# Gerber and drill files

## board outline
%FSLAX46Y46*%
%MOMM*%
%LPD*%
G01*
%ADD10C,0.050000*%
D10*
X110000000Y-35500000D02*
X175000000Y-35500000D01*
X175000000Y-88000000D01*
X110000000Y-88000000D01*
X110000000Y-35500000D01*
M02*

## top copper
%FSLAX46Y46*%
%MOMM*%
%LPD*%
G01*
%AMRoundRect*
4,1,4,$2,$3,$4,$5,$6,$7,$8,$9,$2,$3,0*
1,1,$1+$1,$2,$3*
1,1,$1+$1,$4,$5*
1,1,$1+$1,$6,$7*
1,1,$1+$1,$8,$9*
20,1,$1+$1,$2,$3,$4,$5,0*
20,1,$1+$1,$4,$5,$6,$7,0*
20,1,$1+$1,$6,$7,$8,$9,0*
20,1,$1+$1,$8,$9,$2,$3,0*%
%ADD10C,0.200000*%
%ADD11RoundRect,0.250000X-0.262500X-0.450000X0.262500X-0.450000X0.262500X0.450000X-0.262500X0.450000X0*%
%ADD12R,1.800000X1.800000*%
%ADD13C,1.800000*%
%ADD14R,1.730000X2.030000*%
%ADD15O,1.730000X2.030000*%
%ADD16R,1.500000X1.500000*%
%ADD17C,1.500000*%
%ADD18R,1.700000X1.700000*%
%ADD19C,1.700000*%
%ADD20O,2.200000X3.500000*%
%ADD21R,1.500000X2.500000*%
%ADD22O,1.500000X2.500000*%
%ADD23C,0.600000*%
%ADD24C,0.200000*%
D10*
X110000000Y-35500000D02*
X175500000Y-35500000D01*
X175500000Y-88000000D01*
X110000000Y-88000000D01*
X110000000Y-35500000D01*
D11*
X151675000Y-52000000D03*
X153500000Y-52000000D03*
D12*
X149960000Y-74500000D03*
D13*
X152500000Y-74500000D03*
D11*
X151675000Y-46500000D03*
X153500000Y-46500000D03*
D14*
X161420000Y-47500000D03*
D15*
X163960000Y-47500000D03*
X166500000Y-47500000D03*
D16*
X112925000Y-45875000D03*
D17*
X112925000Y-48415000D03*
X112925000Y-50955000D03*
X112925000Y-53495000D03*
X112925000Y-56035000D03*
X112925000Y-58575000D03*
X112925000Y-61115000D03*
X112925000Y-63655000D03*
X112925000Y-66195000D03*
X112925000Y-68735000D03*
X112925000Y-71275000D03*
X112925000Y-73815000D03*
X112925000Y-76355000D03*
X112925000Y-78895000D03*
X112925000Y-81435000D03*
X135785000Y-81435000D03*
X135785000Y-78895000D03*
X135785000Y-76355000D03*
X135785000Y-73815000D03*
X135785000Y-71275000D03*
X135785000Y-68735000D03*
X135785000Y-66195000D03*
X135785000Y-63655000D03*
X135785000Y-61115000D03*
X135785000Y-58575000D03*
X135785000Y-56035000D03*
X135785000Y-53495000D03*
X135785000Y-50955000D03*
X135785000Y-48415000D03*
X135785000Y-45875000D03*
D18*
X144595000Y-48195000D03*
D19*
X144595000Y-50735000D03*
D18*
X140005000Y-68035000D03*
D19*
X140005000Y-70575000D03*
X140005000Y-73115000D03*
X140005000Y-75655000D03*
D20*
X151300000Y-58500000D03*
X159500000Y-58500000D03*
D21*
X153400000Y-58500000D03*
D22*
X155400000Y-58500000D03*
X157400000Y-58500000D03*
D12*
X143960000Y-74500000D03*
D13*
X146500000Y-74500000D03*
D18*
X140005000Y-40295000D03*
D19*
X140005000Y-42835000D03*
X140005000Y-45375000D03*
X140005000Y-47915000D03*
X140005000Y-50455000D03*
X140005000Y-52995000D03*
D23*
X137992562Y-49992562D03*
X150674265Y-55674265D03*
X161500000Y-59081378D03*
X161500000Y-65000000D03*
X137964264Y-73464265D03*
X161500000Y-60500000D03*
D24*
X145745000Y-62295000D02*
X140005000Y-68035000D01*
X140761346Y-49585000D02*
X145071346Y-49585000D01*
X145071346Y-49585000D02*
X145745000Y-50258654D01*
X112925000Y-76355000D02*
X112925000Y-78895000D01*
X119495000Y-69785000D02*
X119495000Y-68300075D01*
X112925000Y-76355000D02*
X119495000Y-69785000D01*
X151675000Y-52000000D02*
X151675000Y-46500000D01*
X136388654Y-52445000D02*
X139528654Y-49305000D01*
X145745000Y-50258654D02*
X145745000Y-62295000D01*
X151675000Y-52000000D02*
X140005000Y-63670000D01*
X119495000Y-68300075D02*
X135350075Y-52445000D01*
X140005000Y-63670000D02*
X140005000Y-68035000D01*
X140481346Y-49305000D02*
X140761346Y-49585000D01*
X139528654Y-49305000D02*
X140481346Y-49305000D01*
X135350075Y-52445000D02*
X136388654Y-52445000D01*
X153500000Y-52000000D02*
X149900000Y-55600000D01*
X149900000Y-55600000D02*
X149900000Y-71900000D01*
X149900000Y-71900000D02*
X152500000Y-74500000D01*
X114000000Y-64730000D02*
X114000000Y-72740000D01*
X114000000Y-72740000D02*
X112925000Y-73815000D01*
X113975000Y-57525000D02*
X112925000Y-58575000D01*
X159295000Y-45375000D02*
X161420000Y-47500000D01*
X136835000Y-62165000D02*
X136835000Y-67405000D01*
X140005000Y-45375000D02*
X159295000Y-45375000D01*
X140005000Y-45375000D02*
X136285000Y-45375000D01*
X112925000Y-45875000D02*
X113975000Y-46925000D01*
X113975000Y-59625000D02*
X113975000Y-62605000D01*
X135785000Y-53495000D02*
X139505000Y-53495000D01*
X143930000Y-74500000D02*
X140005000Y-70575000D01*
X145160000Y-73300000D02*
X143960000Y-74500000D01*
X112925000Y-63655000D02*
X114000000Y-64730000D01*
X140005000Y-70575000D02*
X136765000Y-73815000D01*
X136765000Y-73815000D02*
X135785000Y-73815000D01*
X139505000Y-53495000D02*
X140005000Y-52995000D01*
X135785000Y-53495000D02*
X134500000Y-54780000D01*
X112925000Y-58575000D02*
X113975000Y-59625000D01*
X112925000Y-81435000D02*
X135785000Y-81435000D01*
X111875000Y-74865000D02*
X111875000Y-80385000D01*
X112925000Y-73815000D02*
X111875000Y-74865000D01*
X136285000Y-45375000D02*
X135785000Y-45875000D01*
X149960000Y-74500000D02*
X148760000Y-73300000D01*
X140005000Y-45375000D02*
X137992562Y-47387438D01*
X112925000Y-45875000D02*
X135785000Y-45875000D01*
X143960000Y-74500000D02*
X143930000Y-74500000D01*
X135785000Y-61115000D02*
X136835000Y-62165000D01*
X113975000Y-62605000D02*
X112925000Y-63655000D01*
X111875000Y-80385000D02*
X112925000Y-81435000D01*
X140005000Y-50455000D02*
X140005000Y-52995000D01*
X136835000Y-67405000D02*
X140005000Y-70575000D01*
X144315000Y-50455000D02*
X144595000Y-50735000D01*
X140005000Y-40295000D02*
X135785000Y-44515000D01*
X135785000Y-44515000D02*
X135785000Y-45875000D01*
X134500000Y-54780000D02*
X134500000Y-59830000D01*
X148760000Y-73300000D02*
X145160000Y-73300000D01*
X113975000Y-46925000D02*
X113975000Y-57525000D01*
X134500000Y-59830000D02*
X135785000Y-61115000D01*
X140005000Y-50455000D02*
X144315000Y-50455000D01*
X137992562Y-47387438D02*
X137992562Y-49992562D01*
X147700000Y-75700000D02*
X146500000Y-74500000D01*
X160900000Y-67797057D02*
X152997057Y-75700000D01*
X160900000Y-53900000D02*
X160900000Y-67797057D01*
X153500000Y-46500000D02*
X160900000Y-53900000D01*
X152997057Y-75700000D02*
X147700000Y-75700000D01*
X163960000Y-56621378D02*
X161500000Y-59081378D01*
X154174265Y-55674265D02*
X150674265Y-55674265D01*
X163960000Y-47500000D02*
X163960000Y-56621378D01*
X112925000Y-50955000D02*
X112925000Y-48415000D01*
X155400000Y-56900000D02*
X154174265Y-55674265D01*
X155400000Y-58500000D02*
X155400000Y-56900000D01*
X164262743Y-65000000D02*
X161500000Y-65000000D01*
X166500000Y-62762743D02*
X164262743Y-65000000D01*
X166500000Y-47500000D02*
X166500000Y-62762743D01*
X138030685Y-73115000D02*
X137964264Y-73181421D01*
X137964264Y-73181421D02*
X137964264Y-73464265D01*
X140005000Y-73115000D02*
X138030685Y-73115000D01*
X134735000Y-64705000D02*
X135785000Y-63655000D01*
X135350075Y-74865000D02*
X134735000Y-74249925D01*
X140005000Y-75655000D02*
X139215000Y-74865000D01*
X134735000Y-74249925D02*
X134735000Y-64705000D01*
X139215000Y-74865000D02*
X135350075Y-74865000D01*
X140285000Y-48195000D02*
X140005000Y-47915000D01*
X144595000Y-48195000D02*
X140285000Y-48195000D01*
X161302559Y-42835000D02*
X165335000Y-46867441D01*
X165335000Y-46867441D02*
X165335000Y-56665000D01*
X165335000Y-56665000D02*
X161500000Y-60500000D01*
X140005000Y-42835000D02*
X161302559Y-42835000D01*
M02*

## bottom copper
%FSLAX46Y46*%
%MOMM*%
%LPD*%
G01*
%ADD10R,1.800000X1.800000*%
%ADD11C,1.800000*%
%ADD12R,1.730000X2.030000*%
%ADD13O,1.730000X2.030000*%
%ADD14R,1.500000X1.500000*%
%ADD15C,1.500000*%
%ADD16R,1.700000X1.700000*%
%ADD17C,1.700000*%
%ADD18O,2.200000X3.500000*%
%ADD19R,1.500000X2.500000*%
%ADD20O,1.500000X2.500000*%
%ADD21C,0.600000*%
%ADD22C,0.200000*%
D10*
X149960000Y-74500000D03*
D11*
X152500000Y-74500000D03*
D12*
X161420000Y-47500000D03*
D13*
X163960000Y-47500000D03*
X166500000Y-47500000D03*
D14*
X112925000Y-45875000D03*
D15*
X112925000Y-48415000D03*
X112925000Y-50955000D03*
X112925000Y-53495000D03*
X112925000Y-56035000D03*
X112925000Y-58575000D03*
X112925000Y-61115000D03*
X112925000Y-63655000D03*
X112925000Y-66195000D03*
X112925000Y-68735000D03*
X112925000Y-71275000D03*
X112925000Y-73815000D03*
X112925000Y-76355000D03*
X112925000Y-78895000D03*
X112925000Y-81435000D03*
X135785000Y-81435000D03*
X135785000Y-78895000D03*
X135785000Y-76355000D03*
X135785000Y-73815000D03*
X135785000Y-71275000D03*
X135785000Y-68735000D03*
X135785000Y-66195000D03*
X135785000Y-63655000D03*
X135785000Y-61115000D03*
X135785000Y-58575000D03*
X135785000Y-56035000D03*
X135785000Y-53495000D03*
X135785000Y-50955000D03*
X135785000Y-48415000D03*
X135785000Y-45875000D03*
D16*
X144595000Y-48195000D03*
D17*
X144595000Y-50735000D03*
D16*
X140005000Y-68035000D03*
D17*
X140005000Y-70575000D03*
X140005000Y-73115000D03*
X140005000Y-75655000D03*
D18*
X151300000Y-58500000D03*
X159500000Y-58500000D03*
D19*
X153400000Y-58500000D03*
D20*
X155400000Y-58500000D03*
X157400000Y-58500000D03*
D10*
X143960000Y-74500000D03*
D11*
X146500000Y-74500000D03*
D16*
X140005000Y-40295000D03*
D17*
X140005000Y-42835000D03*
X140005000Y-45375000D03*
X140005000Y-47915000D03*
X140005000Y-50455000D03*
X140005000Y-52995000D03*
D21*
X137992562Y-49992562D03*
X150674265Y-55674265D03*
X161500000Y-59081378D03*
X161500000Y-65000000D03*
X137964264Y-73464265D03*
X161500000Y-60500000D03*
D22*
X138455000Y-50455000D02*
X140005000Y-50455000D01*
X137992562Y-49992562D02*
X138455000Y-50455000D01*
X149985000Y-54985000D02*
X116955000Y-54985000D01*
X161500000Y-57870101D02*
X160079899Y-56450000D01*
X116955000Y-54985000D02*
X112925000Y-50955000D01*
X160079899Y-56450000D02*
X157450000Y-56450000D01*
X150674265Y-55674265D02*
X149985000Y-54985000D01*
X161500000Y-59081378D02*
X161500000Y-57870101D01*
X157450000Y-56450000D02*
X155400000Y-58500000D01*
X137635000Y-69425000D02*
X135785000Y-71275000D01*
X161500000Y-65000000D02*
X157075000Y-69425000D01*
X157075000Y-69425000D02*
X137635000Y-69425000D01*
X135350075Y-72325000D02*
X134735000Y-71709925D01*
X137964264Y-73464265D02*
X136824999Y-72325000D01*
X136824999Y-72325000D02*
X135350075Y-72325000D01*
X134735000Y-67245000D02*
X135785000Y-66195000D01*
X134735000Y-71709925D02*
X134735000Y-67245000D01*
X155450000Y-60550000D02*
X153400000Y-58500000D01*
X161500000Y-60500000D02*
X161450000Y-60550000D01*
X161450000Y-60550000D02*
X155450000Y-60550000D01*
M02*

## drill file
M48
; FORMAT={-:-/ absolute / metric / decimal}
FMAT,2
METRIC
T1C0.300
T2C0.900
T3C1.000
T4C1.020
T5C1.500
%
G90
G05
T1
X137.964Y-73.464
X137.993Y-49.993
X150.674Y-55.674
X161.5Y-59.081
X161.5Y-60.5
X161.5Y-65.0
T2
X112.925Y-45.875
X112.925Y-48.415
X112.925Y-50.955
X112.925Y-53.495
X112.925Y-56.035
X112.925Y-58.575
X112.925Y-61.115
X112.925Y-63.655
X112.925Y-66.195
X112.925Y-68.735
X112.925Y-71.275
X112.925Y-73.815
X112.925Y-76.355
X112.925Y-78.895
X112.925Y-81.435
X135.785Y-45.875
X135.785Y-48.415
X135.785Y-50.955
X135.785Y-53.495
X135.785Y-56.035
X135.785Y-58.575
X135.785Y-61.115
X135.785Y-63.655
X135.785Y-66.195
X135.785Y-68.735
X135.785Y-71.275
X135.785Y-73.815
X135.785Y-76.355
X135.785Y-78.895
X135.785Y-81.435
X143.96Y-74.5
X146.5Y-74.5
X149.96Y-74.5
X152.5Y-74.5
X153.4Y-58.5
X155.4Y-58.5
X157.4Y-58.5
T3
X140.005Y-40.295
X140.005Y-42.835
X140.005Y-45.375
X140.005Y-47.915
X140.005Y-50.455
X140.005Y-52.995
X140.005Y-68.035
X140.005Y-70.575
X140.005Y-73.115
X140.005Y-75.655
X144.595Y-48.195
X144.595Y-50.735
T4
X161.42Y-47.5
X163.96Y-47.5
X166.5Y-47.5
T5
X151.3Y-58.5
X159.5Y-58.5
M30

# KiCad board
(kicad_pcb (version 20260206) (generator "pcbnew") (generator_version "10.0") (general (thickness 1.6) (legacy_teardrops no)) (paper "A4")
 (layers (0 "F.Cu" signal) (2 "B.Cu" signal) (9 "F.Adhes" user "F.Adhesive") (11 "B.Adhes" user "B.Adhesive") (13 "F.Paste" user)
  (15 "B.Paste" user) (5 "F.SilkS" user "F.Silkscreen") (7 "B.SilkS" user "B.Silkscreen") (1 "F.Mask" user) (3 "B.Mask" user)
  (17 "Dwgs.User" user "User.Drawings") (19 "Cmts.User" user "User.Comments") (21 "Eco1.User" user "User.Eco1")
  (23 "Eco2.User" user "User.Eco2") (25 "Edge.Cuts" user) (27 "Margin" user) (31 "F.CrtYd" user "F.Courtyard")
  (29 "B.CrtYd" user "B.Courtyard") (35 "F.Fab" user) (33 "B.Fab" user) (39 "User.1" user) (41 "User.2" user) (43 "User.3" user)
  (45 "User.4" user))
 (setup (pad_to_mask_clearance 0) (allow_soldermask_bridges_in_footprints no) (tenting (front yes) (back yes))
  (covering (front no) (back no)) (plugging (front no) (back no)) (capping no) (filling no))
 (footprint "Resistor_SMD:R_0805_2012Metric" (layer "F.Cu") (at 152.5875 52)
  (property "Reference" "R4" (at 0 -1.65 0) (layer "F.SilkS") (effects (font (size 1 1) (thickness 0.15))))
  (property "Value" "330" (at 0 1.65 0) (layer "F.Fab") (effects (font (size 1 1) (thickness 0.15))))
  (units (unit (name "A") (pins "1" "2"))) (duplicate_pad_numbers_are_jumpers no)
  (pad "1" smd roundrect (at -0.9125 0) (size 1.025 1.4) (layers "F.Cu" "F.Mask" "F.Paste") (roundrect_rratio 0.243902) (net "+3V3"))
  (pad "2" smd roundrect (at 0.9125 0) (size 1.025 1.4) (layers "F.Cu" "F.Mask" "F.Paste") (roundrect_rratio 0.243902) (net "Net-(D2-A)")))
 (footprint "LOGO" (layer "F.Cu") (at 161.5 79)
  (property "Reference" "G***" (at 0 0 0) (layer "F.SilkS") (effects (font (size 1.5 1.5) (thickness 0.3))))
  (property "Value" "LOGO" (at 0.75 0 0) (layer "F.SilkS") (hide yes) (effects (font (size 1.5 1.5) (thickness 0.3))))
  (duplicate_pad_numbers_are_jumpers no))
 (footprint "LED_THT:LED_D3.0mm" (layer "F.Cu") (at 149.96 74.5)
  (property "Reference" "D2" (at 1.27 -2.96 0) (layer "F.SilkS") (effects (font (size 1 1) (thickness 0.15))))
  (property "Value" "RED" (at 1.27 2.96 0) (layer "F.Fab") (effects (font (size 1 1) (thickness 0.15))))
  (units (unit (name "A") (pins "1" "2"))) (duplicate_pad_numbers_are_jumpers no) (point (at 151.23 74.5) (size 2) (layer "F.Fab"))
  (pad "1" thru_hole rect (at 0 0) (size 1.8 1.8) (drill 0.9) (layers "*.Cu" "*.Mask") (remove_unused_layers no) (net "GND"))
  (pad "2" thru_hole circle (at 2.54 0) (size 1.8 1.8) (drill 0.9) (layers "*.Cu" "*.Mask") (remove_unused_layers no) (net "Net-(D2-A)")))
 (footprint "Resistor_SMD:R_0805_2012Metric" (layer "F.Cu") (at 152.5875 46.5)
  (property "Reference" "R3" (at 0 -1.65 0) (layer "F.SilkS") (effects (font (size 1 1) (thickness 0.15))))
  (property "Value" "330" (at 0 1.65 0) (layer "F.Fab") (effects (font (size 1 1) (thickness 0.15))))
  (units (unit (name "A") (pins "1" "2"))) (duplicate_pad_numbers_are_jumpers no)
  (pad "1" smd roundrect (at -0.9125 0) (size 1.025 1.4) (layers "F.Cu" "F.Mask" "F.Paste") (roundrect_rratio 0.243902) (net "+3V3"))
  (pad "2" smd roundrect (at 0.9125 0) (size 1.025 1.4) (layers "F.Cu" "F.Mask" "F.Paste") (roundrect_rratio 0.243902) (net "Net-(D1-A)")))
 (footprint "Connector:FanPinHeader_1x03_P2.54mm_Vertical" (layer "F.Cu") (at 161.42 47.5)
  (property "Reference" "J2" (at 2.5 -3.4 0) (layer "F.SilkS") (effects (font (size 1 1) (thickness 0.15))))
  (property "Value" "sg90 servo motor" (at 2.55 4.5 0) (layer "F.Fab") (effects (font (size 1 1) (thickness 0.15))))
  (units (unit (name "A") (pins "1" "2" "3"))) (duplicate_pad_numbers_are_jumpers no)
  (pad "1" thru_hole rect (at 0 0 90) (size 2.03 1.73) (drill 1.02) (layers "*.Cu" "*.Mask") (remove_unused_layers no) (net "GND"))
  (pad "2" thru_hole oval (at 2.54 0 90) (size 2.03 1.73) (drill 1.02) (layers "*.Cu" "*.Mask") (remove_unused_layers no) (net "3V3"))
  (pad "3" thru_hole oval (at 5.08 0 90) (size 2.03 1.73) (drill 1.02) (layers "*.Cu" "*.Mask") (remove_unused_layers no)
   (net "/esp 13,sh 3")))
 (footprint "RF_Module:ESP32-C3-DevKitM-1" (layer "F.Cu") (at 112.925 45.875)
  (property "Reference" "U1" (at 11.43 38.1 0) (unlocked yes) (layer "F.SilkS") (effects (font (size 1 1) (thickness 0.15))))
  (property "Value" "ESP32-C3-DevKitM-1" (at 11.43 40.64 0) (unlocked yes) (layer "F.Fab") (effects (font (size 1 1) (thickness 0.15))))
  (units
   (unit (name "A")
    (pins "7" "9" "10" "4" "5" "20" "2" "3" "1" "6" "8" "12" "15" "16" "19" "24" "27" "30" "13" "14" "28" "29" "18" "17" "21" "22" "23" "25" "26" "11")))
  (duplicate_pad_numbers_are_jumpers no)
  (pad "1" thru_hole rect (at 0 0) (size 1.5 1.5) (drill 0.9) (layers "*.Cu" "*.Mask") (remove_unused_layers yes) (keep_end_layers yes)
   (zone_layer_connections) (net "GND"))
  (pad "2" thru_hole circle (at 0 2.54) (size 1.5 1.5) (drill 0.9) (layers "*.Cu" "*.Mask") (remove_unused_layers yes) (keep_end_layers yes)
   (zone_layer_connections) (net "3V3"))
  (pad "3" thru_hole circle (at 0 5.08) (size 1.5 1.5) (drill 0.9) (layers "*.Cu" "*.Mask") (remove_unused_layers yes) (keep_end_layers yes)
   (zone_layer_connections) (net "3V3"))
  (pad "4" thru_hole circle (at 0 7.62) (size 1.5 1.5) (drill 0.9) (layers "*.Cu" "*.Mask") (remove_unused_layers yes) (keep_end_layers yes)
   (zone_layer_connections) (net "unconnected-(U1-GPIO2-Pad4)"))
  (pad "5" thru_hole circle (at 0 10.16) (size 1.5 1.5) (drill 0.9) (layers "*.Cu" "*.Mask") (remove_unused_layers yes)
   (keep_end_layers yes) (zone_layer_connections) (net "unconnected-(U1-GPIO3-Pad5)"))
  (pad "6" thru_hole circle (at 0 12.7) (size 1.5 1.5) (drill 0.9) (layers "*.Cu" "*.Mask") (remove_unused_layers yes) (keep_end_layers yes)
   (zone_layer_connections) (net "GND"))
  (pad "7" thru_hole circle (at 0 15.24) (size 1.5 1.5) (drill 0.9) (layers "*.Cu" "*.Mask") (remove_unused_layers yes)
   (keep_end_layers yes) (zone_layer_connections) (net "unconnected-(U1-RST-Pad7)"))
  (pad "8" thru_hole circle (at 0 17.78) (size 1.5 1.5) (drill 0.9) (layers "*.Cu" "*.Mask") (remove_unused_layers yes)
   (keep_end_layers yes) (zone_layer_connections) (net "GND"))
  (pad "9" thru_hole circle (at 0 20.32) (size 1.5 1.5) (drill 0.9) (layers "*.Cu" "*.Mask") (remove_unused_layers yes)
   (keep_end_layers yes) (zone_layer_connections) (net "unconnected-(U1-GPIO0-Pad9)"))
  (pad "10" thru_hole circle (at 0 22.86) (size 1.5 1.5) (drill 0.9) (layers "*.Cu" "*.Mask") (remove_unused_layers yes)
   (keep_end_layers yes) (zone_layer_connections) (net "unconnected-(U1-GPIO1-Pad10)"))
  (pad "11" thru_hole circle (at 0 25.4) (size 1.5 1.5) (drill 0.9) (layers "*.Cu" "*.Mask") (remove_unused_layers yes)
   (keep_end_layers yes) (zone_layer_connections) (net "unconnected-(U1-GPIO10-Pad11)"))
  (pad "12" thru_hole circle (at 0 27.94) (size 1.5 1.5) (drill 0.9) (layers "*.Cu" "*.Mask") (remove_unused_layers yes)
   (keep_end_layers yes) (zone_layer_connections) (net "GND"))
  (pad "13" thru_hole circle (at 0 30.48) (size 1.5 1.5) (drill 0.9) (layers "*.Cu" "*.Mask") (remove_unused_layers yes)
   (keep_end_layers yes) (zone_layer_connections) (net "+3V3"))
  (pad "14" thru_hole circle (at 0 33.02) (size 1.5 1.5) (drill 0.9) (layers "*.Cu" "*.Mask") (remove_unused_layers yes)
   (keep_end_layers yes) (zone_layer_connections) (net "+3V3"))
  (pad "15" thru_hole circle (at 0 35.56) (size 1.5 1.5) (drill 0.9) (layers "*.Cu" "*.Mask") (remove_unused_layers yes)
   (keep_end_layers yes) (zone_layer_connections) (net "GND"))
  (pad "16" thru_hole circle (at 22.86 35.56) (size 1.5 1.5) (drill 0.9) (layers "*.Cu" "*.Mask") (remove_unused_layers yes)
   (keep_end_layers yes) (zone_layer_connections) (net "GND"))
  (pad "17" thru_hole circle (at 22.86 33.02) (size 1.5 1.5) (drill 0.9) (layers "*.Cu" "*.Mask") (remove_unused_layers yes)
   (keep_end_layers yes) (zone_layer_connections) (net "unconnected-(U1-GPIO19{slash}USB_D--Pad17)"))
  (pad "18" thru_hole circle (at 22.86 30.48) (size 1.5 1.5) (drill 0.9) (layers "*.Cu" "*.Mask") (remove_unused_layers yes)
   (keep_end_layers yes) (zone_layer_connections) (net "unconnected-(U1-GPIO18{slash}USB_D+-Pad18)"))
  (pad "19" thru_hole circle (at 22.86 27.94) (size 1.5 1.5) (drill 0.9) (layers "*.Cu" "*.Mask") (remove_unused_layers yes)
   (keep_end_layers yes) (zone_layer_connections) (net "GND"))
  (pad "20" thru_hole circle (at 22.86 25.4) (size 1.5 1.5) (drill 0.9) (layers "*.Cu" "*.Mask") (remove_unused_layers yes)
   (keep_end_layers yes) (zone_layer_connections) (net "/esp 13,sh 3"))
  (pad "21" thru_hole circle (at 22.86 22.86) (size 1.5 1.5) (drill 0.9) (layers "*.Cu" "*.Mask") (remove_unused_layers yes)
   (keep_end_layers yes) (zone_layer_connections) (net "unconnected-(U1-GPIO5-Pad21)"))
  (pad "22" thru_hole circle (at 22.86 20.32) (size 1.5 1.5) (drill 0.9) (layers "*.Cu" "*.Mask") (remove_unused_layers yes)
   (keep_end_layers yes) (zone_layer_connections) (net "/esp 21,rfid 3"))
  (pad "23" thru_hole circle (at 22.86 17.78) (size 1.5 1.5) (drill 0.9) (layers "*.Cu" "*.Mask") (remove_unused_layers yes)
   (keep_end_layers yes) (zone_layer_connections) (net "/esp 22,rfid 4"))
  (pad "24" thru_hole circle (at 22.86 15.24) (size 1.5 1.5) (drill 0.9) (layers "*.Cu" "*.Mask") (remove_unused_layers yes)
   (keep_end_layers yes) (zone_layer_connections) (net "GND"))
  (pad "25" thru_hole circle (at 22.86 12.7) (size 1.5 1.5) (drill 0.9) (layers "*.Cu" "*.Mask") (remove_unused_layers yes)
   (keep_end_layers yes) (zone_layer_connections) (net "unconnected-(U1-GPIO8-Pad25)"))
  (pad "26" thru_hole circle (at 22.86 10.16) (size 1.5 1.5) (drill 0.9) (layers "*.Cu" "*.Mask") (remove_unused_layers yes)
   (keep_end_layers yes) (zone_layer_connections) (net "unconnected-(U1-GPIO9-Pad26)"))
  (pad "27" thru_hole circle (at 22.86 7.62) (size 1.5 1.5) (drill 0.9) (layers "*.Cu" "*.Mask") (remove_unused_layers yes)
   (keep_end_layers yes) (zone_layer_connections) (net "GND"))
  (pad "28" thru_hole circle (at 22.86 5.08) (size 1.5 1.5) (drill 0.9) (layers "*.Cu" "*.Mask") (remove_unused_layers yes)
   (keep_end_layers yes) (zone_layer_connections) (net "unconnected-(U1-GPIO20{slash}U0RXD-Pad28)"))
  (pad "29" thru_hole circle (at 22.86 2.54) (size 1.5 1.5) (drill 0.9) (layers "*.Cu" "*.Mask") (remove_unused_layers yes)
   (keep_end_layers yes) (zone_layer_connections) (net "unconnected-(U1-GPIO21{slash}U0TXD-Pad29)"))
  (pad "30" thru_hole circle (at 22.86 0) (size 1.5 1.5) (drill 0.9) (layers "*.Cu" "*.Mask") (remove_unused_layers yes)
   (keep_end_layers yes) (zone_layer_connections) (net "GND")))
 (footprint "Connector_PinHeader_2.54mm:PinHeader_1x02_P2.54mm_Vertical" (layer "F.Cu") (at 144.595 48.195)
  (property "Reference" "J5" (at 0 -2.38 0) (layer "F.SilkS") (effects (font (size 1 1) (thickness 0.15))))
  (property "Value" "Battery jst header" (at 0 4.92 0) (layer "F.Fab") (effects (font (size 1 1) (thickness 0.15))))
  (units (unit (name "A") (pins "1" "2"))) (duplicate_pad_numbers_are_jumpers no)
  (pad "1" thru_hole rect (at 0 0) (size 1.7 1.7) (drill 1) (layers "*.Cu" "*.Mask") (remove_unused_layers no) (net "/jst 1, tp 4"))
  (pad "2" thru_hole circle (at 0 2.54) (size 1.7 1.7) (drill 1) (layers "*.Cu" "*.Mask") (remove_unused_layers no) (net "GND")))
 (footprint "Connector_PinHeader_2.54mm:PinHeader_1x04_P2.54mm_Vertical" (layer "F.Cu") (at 140.005 68.035)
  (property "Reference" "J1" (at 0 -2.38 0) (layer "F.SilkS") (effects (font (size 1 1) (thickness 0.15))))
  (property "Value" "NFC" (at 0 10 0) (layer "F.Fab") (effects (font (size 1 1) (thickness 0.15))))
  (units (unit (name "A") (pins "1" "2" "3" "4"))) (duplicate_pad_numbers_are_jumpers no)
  (pad "1" thru_hole rect (at 0 0) (size 1.7 1.7) (drill 1) (layers "*.Cu" "*.Mask") (remove_unused_layers no) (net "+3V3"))
  (pad "2" thru_hole circle (at 0 2.54) (size 1.7 1.7) (drill 1) (layers "*.Cu" "*.Mask") (remove_unused_layers no) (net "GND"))
  (pad "3" thru_hole circle (at 0 5.08) (size 1.7 1.7) (drill 1) (layers "*.Cu" "*.Mask") (remove_unused_layers no) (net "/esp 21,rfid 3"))
  (pad "4" thru_hole circle (at 0 7.62) (size 1.7 1.7) (drill 1) (layers "*.Cu" "*.Mask") (remove_unused_layers no) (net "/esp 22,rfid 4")))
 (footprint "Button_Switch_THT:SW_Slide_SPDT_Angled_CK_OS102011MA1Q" (layer "F.Cu") (at 153.4 58.5)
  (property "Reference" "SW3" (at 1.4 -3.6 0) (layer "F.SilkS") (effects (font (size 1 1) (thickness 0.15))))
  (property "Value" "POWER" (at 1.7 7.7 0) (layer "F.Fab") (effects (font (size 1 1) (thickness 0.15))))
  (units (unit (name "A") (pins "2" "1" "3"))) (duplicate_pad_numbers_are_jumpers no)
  (pad "" thru_hole oval (at -2.1 0) (size 2.2 3.5) (drill 1.5) (layers "*.Cu" "*.Mask") (remove_unused_layers no))
  (pad "" thru_hole oval (at 6.1 0) (size 2.2 3.5) (drill 1.5) (layers "*.Cu" "*.Mask") (remove_unused_layers no))
  (pad "1" thru_hole rect (at 0 0) (size 1.5 2.5) (drill 0.9) (layers "*.Cu" "*.Mask") (remove_unused_layers no) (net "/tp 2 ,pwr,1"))
  (pad "2" thru_hole oval (at 2 0) (size 1.5 2.5) (drill 0.9) (layers "*.Cu" "*.Mask") (remove_unused_layers no) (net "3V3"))
  (pad "3" thru_hole oval (at 4 0) (size 1.5 2.5) (drill 0.9) (layers "*.Cu" "*.Mask") (remove_unused_layers no)
   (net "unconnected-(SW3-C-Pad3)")))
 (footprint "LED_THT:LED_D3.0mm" (layer "F.Cu") (at 143.96 74.5)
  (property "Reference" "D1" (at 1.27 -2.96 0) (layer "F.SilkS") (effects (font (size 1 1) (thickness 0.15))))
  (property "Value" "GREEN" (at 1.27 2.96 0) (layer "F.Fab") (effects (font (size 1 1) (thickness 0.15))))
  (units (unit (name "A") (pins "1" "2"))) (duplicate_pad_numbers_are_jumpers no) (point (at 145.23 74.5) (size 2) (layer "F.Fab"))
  (pad "1" thru_hole rect (at 0 0) (size 1.8 1.8) (drill 0.9) (layers "*.Cu" "*.Mask") (remove_unused_layers no) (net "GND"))
  (pad "2" thru_hole circle (at 2.54 0) (size 1.8 1.8) (drill 0.9) (layers "*.Cu" "*.Mask") (remove_unused_layers no) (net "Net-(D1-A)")))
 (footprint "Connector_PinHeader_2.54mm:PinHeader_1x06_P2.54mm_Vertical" (layer "F.Cu") (at 140.005 40.295)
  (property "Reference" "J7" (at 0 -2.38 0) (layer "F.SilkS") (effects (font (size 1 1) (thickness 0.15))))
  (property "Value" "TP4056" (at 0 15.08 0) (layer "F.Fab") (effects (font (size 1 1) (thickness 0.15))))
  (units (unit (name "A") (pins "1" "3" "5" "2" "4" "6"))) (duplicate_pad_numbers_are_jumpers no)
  (pad "1" thru_hole rect (at 0 0) (size 1.7 1.7) (drill 1) (layers "*.Cu" "*.Mask") (remove_unused_layers no) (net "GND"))
  (pad "2" thru_hole circle (at 0 2.54) (size 1.7 1.7) (drill 1) (layers "*.Cu" "*.Mask") (remove_unused_layers no) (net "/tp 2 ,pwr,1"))
  (pad "3" thru_hole circle (at 0 5.08) (size 1.7 1.7) (drill 1) (layers "*.Cu" "*.Mask") (remove_unused_layers no) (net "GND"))
  (pad "4" thru_hole circle (at 0 7.62) (size 1.7 1.7) (drill 1) (layers "*.Cu" "*.Mask") (remove_unused_layers no) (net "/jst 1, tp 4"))
  (pad "5" thru_hole circle (at 0 10.16) (size 1.7 1.7) (drill 1) (layers "*.Cu" "*.Mask") (remove_unused_layers no) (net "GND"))
  (pad "6" thru_hole circle (at 0 12.7) (size 1.7 1.7) (drill 1) (layers "*.Cu" "*.Mask") (remove_unused_layers no) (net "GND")))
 (gr_rect (start 110 35.5) (end 175.5 88) (stroke (width 0.2) (type default)) (fill no) (layer "F.Cu"))
 (gr_rect (start 110 35.5) (end 175 88) (stroke (width 0.05) (type default)) (fill no) (layer "Edge.Cuts"))
 (segment (start 145.745 62.295) (end 140.005 68.035) (width 0.2) (layer "F.Cu") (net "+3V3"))
 (segment (start 140.761346 49.585) (end 145.071346 49.585) (width 0.2) (layer "F.Cu") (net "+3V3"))
 (segment (start 145.071346 49.585) (end 145.745 50.258654) (width 0.2) (layer "F.Cu") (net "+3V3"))
 (segment (start 112.925 76.355) (end 112.925 78.895) (width 0.2) (layer "F.Cu") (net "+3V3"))
 (segment (start 119.495 69.785) (end 119.495 68.300075) (width 0.2) (layer "F.Cu") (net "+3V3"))
 (segment (start 112.925 76.355) (end 119.495 69.785) (width 0.2) (layer "F.Cu") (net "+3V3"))
 (segment (start 151.675 52) (end 151.675 46.5) (width 0.2) (layer "F.Cu") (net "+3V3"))
 (segment (start 136.388654 52.445) (end 139.528654 49.305) (width 0.2) (layer "F.Cu") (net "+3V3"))
 (segment (start 145.745 50.258654) (end 145.745 62.295) (width 0.2) (layer "F.Cu") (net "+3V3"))
 (segment (start 151.675 52) (end 140.005 63.67) (width 0.2) (layer "F.Cu") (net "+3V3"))
 (segment (start 119.495 68.300075) (end 135.350075 52.445) (width 0.2) (layer "F.Cu") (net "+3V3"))
 (segment (start 140.005 63.67) (end 140.005 68.035) (width 0.2) (layer "F.Cu") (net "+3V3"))
 (segment (start 140.481346 49.305) (end 140.761346 49.585) (width 0.2) (layer "F.Cu") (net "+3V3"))
 (segment (start 139.528654 49.305) (end 140.481346 49.305) (width 0.2) (layer "F.Cu") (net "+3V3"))
 (segment (start 135.350075 52.445) (end 136.388654 52.445) (width 0.2) (layer "F.Cu") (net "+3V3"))
 (segment (start 153.5 52) (end 149.9 55.6) (width 0.2) (layer "F.Cu") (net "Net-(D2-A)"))
 (segment (start 149.9 55.6) (end 149.9 71.9) (width 0.2) (layer "F.Cu") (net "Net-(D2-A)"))
 (segment (start 149.9 71.9) (end 152.5 74.5) (width 0.2) (layer "F.Cu") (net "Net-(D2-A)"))
 (segment (start 114 64.73) (end 114 72.74) (width 0.2) (layer "F.Cu") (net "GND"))
 (segment (start 114 72.74) (end 112.925 73.815) (width 0.2) (layer "F.Cu") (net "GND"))
 (segment (start 113.975 57.525) (end 112.925 58.575) (width 0.2) (layer "F.Cu") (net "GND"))
 (segment (start 159.295 45.375) (end 161.42 47.5) (width 0.2) (layer "F.Cu") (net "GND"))
 (segment (start 136.835 62.165) (end 136.835 67.405) (width 0.2) (layer "F.Cu") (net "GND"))
 (segment (start 140.005 45.375) (end 159.295 45.375) (width 0.2) (layer "F.Cu") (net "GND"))
 (segment (start 140.005 45.375) (end 136.285 45.375) (width 0.2) (layer "F.Cu") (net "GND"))
 (segment (start 112.925 45.875) (end 113.975 46.925) (width 0.2) (layer "F.Cu") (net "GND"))
 (segment (start 113.975 59.625) (end 113.975 62.605) (width 0.2) (layer "F.Cu") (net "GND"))
 (segment (start 135.785 53.495) (end 139.505 53.495) (width 0.2) (layer "F.Cu") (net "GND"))
 (segment (start 143.93 74.5) (end 140.005 70.575) (width 0.2) (layer "F.Cu") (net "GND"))
 (segment (start 145.16 73.3) (end 143.96 74.5) (width 0.2) (layer "F.Cu") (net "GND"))
 (segment (start 112.925 63.655) (end 114 64.73) (width 0.2) (layer "F.Cu") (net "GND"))
 (segment (start 140.005 70.575) (end 136.765 73.815) (width 0.2) (layer "F.Cu") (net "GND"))
 (segment (start 136.765 73.815) (end 135.785 73.815) (width 0.2) (layer "F.Cu") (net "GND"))
 (segment (start 139.505 53.495) (end 140.005 52.995) (width 0.2) (layer "F.Cu") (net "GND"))
 (segment (start 135.785 53.495) (end 134.5 54.78) (width 0.2) (layer "F.Cu") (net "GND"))
 (segment (start 112.925 58.575) (end 113.975 59.625) (width 0.2) (layer "F.Cu") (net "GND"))
 (segment (start 112.925 81.435) (end 135.785 81.435) (width 0.2) (layer "F.Cu") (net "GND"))
 (segment (start 111.875 74.865) (end 111.875 80.385) (width 0.2) (layer "F.Cu") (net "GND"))
 (segment (start 112.925 73.815) (end 111.875 74.865) (width 0.2) (layer "F.Cu") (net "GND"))
 (segment (start 136.285 45.375) (end 135.785 45.875) (width 0.2) (layer "F.Cu") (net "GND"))
 (segment (start 149.96 74.5) (end 148.76 73.3) (width 0.2) (layer "F.Cu") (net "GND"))
 (segment (start 140.005 45.375) (end 137.992562 47.387438) (width 0.2) (layer "F.Cu") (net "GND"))
 (segment (start 112.925 45.875) (end 135.785 45.875) (width 0.2) (layer "F.Cu") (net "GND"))
 (segment (start 143.96 74.5) (end 143.93 74.5) (width 0.2) (layer "F.Cu") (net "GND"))
 (segment (start 135.785 61.115) (end 136.835 62.165) (width 0.2) (layer "F.Cu") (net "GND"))
 (segment (start 113.975 62.605) (end 112.925 63.655) (width 0.2) (layer "F.Cu") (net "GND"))
 (segment (start 111.875 80.385) (end 112.925 81.435) (width 0.2) (layer "F.Cu") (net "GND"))
 (segment (start 140.005 50.455) (end 140.005 52.995) (width 0.2) (layer "F.Cu") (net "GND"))
 (segment (start 136.835 67.405) (end 140.005 70.575) (width 0.2) (layer "F.Cu") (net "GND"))
 (segment (start 144.315 50.455) (end 144.595 50.735) (width 0.2) (layer "F.Cu") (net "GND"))
 (segment (start 140.005 40.295) (end 135.785 44.515) (width 0.2) (layer "F.Cu") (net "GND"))
 (segment (start 135.785 44.515) (end 135.785 45.875) (width 0.2) (layer "F.Cu") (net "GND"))
 (segment (start 134.5 54.78) (end 134.5 59.83) (width 0.2) (layer "F.Cu") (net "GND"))
 (segment (start 148.76 73.3) (end 145.16 73.3) (width 0.2) (layer "F.Cu") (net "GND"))
 (segment (start 113.975 46.925) (end 113.975 57.525) (width 0.2) (layer "F.Cu") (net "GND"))
 (segment (start 134.5 59.83) (end 135.785 61.115) (width 0.2) (layer "F.Cu") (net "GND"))
 (segment (start 140.005 50.455) (end 144.315 50.455) (width 0.2) (layer "F.Cu") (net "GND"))
 (segment (start 137.992562 47.387438) (end 137.992562 49.992562) (width 0.2) (layer "F.Cu") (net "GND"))
 (via (at 137.992562 49.992562) (size 0.6) (drill 0.3) (layers "F.Cu" "B.Cu") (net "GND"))
 (segment (start 138.455 50.455) (end 140.005 50.455) (width 0.2) (layer "B.Cu") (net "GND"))
 (segment (start 137.992562 49.992562) (end 138.455 50.455) (width 0.2) (layer "B.Cu") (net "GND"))
 (segment (start 147.7 75.7) (end 146.5 74.5) (width 0.2) (layer "F.Cu") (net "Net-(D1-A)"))
 (segment (start 160.9 67.797057) (end 152.997057 75.7) (width 0.2) (layer "F.Cu") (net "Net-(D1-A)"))
 (segment (start 160.9 53.9) (end 160.9 67.797057) (width 0.2) (layer "F.Cu") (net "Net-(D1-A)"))
 (segment (start 153.5 46.5) (end 160.9 53.9) (width 0.2) (layer "F.Cu") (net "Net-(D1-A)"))
 (segment (start 152.997057 75.7) (end 147.7 75.7) (width 0.2) (layer "F.Cu") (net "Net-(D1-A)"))
 (segment (start 163.96 56.621378) (end 161.5 59.081378) (width 0.2) (layer "F.Cu") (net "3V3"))
 (segment (start 154.174265 55.674265) (end 150.674265 55.674265) (width 0.2) (layer "F.Cu") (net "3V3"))
 (segment (start 163.96 47.5) (end 163.96 56.621378) (width 0.2) (layer "F.Cu") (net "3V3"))
 (segment (start 112.925 50.955) (end 112.925 48.415) (width 0.2) (layer "F.Cu") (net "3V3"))
 (segment (start 155.4 56.9) (end 154.174265 55.674265) (width 0.2) (layer "F.Cu") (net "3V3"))
 (segment (start 155.4 58.5) (end 155.4 56.9) (width 0.2) (layer "F.Cu") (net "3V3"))
 (via (at 150.674265 55.674265) (size 0.6) (drill 0.3) (layers "F.Cu" "B.Cu") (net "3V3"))
 (via (at 161.5 59.081378) (size 0.6) (drill 0.3) (layers "F.Cu" "B.Cu") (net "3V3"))
 (segment (start 149.985 54.985) (end 116.955 54.985) (width 0.2) (layer "B.Cu") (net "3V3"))
 (segment (start 161.5 57.870101) (end 160.079899 56.45) (width 0.2) (layer "B.Cu") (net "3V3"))
 (segment (start 116.955 54.985) (end 112.925 50.955) (width 0.2) (layer "B.Cu") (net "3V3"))
 (segment (start 160.079899 56.45) (end 157.45 56.45) (width 0.2) (layer "B.Cu") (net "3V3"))
 (segment (start 150.674265 55.674265) (end 149.985 54.985) (width 0.2) (layer "B.Cu") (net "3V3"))
 (segment (start 161.5 59.081378) (end 161.5 57.870101) (width 0.2) (layer "B.Cu") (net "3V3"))
 (segment (start 157.45 56.45) (end 155.4 58.5) (width 0.2) (layer "B.Cu") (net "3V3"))
 (segment (start 164.262743 65) (end 161.5 65) (width 0.2) (layer "F.Cu") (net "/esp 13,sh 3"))
 (segment (start 166.5 62.762743) (end 164.262743 65) (width 0.2) (layer "F.Cu") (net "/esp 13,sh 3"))
 (segment (start 166.5 47.5) (end 166.5 62.762743) (width 0.2) (layer "F.Cu") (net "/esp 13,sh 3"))
 (via (at 161.5 65) (size 0.6) (drill 0.3) (layers "F.Cu" "B.Cu") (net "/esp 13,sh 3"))
 (segment (start 137.635 69.425) (end 135.785 71.275) (width 0.2) (layer "B.Cu") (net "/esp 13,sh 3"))
 (segment (start 161.5 65) (end 157.075 69.425) (width 0.2) (layer "B.Cu") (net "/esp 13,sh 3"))
 (segment (start 157.075 69.425) (end 137.635 69.425) (width 0.2) (layer "B.Cu") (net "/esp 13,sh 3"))
 (segment (start 138.030685 73.115) (end 137.964264 73.181421) (width 0.2) (layer "F.Cu") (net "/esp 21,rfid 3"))
 (segment (start 137.964264 73.181421) (end 137.964264 73.464265) (width 0.2) (layer "F.Cu") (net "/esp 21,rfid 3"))
 (segment (start 140.005 73.115) (end 138.030685 73.115) (width 0.2) (layer "F.Cu") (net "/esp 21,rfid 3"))
 (via (at 137.964264 73.464265) (size 0.6) (drill 0.3) (layers "F.Cu" "B.Cu") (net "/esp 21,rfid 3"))
 (segment (start 135.350075 72.325) (end 134.735 71.709925) (width 0.2) (layer "B.Cu") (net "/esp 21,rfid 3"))
 (segment (start 137.964264 73.464265) (end 136.824999 72.325) (width 0.2) (layer "B.Cu") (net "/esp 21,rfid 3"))
 (segment (start 136.824999 72.325) (end 135.350075 72.325) (width 0.2) (layer "B.Cu") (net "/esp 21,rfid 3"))
 (segment (start 134.735 67.245) (end 135.785 66.195) (width 0.2) (layer "B.Cu") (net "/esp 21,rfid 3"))
 (segment (start 134.735 71.709925) (end 134.735 67.245) (width 0.2) (layer "B.Cu") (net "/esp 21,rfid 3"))
 (segment (start 134.735 64.705) (end 135.785 63.655) (width 0.2) (layer "F.Cu") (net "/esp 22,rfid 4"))
 (segment (start 135.350075 74.865) (end 134.735 74.249925) (width 0.2) (layer "F.Cu") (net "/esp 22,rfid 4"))
 (segment (start 140.005 75.655) (end 139.215 74.865) (width 0.2) (layer "F.Cu") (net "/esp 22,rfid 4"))
 (segment (start 134.735 74.249925) (end 134.735 64.705) (width 0.2) (layer "F.Cu") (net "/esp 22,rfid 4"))
 (segment (start 139.215 74.865) (end 135.350075 74.865) (width 0.2) (layer "F.Cu") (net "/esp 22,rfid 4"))
 (segment (start 140.285 48.195) (end 140.005 47.915) (width 0.2) (layer "F.Cu") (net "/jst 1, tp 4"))
 (segment (start 144.595 48.195) (end 140.285 48.195) (width 0.2) (layer "F.Cu") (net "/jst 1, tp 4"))
 (segment (start 161.302559 42.835) (end 165.335 46.867441) (width 0.2) (layer "F.Cu") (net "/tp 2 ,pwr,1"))
 (segment (start 165.335 46.867441) (end 165.335 56.665) (width 0.2) (layer "F.Cu") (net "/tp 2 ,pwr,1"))
 (segment (start 165.335 56.665) (end 161.5 60.5) (width 0.2) (layer "F.Cu") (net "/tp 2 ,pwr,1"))
 (segment (start 140.005 42.835) (end 161.302559 42.835) (width 0.2) (layer "F.Cu") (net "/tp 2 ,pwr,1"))
 (via (at 161.5 60.5) (size 0.6) (drill 0.3) (layers "F.Cu" "B.Cu") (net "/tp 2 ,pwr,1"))
 (segment (start 155.45 60.55) (end 153.4 58.5) (width 0.2) (layer "B.Cu") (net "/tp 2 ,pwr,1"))
 (segment (start 161.5 60.5) (end 161.45 60.55) (width 0.2) (layer "B.Cu") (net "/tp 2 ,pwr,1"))
 (segment (start 161.45 60.55) (end 155.45 60.55) (width 0.2) (layer "B.Cu") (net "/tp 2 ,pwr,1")))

